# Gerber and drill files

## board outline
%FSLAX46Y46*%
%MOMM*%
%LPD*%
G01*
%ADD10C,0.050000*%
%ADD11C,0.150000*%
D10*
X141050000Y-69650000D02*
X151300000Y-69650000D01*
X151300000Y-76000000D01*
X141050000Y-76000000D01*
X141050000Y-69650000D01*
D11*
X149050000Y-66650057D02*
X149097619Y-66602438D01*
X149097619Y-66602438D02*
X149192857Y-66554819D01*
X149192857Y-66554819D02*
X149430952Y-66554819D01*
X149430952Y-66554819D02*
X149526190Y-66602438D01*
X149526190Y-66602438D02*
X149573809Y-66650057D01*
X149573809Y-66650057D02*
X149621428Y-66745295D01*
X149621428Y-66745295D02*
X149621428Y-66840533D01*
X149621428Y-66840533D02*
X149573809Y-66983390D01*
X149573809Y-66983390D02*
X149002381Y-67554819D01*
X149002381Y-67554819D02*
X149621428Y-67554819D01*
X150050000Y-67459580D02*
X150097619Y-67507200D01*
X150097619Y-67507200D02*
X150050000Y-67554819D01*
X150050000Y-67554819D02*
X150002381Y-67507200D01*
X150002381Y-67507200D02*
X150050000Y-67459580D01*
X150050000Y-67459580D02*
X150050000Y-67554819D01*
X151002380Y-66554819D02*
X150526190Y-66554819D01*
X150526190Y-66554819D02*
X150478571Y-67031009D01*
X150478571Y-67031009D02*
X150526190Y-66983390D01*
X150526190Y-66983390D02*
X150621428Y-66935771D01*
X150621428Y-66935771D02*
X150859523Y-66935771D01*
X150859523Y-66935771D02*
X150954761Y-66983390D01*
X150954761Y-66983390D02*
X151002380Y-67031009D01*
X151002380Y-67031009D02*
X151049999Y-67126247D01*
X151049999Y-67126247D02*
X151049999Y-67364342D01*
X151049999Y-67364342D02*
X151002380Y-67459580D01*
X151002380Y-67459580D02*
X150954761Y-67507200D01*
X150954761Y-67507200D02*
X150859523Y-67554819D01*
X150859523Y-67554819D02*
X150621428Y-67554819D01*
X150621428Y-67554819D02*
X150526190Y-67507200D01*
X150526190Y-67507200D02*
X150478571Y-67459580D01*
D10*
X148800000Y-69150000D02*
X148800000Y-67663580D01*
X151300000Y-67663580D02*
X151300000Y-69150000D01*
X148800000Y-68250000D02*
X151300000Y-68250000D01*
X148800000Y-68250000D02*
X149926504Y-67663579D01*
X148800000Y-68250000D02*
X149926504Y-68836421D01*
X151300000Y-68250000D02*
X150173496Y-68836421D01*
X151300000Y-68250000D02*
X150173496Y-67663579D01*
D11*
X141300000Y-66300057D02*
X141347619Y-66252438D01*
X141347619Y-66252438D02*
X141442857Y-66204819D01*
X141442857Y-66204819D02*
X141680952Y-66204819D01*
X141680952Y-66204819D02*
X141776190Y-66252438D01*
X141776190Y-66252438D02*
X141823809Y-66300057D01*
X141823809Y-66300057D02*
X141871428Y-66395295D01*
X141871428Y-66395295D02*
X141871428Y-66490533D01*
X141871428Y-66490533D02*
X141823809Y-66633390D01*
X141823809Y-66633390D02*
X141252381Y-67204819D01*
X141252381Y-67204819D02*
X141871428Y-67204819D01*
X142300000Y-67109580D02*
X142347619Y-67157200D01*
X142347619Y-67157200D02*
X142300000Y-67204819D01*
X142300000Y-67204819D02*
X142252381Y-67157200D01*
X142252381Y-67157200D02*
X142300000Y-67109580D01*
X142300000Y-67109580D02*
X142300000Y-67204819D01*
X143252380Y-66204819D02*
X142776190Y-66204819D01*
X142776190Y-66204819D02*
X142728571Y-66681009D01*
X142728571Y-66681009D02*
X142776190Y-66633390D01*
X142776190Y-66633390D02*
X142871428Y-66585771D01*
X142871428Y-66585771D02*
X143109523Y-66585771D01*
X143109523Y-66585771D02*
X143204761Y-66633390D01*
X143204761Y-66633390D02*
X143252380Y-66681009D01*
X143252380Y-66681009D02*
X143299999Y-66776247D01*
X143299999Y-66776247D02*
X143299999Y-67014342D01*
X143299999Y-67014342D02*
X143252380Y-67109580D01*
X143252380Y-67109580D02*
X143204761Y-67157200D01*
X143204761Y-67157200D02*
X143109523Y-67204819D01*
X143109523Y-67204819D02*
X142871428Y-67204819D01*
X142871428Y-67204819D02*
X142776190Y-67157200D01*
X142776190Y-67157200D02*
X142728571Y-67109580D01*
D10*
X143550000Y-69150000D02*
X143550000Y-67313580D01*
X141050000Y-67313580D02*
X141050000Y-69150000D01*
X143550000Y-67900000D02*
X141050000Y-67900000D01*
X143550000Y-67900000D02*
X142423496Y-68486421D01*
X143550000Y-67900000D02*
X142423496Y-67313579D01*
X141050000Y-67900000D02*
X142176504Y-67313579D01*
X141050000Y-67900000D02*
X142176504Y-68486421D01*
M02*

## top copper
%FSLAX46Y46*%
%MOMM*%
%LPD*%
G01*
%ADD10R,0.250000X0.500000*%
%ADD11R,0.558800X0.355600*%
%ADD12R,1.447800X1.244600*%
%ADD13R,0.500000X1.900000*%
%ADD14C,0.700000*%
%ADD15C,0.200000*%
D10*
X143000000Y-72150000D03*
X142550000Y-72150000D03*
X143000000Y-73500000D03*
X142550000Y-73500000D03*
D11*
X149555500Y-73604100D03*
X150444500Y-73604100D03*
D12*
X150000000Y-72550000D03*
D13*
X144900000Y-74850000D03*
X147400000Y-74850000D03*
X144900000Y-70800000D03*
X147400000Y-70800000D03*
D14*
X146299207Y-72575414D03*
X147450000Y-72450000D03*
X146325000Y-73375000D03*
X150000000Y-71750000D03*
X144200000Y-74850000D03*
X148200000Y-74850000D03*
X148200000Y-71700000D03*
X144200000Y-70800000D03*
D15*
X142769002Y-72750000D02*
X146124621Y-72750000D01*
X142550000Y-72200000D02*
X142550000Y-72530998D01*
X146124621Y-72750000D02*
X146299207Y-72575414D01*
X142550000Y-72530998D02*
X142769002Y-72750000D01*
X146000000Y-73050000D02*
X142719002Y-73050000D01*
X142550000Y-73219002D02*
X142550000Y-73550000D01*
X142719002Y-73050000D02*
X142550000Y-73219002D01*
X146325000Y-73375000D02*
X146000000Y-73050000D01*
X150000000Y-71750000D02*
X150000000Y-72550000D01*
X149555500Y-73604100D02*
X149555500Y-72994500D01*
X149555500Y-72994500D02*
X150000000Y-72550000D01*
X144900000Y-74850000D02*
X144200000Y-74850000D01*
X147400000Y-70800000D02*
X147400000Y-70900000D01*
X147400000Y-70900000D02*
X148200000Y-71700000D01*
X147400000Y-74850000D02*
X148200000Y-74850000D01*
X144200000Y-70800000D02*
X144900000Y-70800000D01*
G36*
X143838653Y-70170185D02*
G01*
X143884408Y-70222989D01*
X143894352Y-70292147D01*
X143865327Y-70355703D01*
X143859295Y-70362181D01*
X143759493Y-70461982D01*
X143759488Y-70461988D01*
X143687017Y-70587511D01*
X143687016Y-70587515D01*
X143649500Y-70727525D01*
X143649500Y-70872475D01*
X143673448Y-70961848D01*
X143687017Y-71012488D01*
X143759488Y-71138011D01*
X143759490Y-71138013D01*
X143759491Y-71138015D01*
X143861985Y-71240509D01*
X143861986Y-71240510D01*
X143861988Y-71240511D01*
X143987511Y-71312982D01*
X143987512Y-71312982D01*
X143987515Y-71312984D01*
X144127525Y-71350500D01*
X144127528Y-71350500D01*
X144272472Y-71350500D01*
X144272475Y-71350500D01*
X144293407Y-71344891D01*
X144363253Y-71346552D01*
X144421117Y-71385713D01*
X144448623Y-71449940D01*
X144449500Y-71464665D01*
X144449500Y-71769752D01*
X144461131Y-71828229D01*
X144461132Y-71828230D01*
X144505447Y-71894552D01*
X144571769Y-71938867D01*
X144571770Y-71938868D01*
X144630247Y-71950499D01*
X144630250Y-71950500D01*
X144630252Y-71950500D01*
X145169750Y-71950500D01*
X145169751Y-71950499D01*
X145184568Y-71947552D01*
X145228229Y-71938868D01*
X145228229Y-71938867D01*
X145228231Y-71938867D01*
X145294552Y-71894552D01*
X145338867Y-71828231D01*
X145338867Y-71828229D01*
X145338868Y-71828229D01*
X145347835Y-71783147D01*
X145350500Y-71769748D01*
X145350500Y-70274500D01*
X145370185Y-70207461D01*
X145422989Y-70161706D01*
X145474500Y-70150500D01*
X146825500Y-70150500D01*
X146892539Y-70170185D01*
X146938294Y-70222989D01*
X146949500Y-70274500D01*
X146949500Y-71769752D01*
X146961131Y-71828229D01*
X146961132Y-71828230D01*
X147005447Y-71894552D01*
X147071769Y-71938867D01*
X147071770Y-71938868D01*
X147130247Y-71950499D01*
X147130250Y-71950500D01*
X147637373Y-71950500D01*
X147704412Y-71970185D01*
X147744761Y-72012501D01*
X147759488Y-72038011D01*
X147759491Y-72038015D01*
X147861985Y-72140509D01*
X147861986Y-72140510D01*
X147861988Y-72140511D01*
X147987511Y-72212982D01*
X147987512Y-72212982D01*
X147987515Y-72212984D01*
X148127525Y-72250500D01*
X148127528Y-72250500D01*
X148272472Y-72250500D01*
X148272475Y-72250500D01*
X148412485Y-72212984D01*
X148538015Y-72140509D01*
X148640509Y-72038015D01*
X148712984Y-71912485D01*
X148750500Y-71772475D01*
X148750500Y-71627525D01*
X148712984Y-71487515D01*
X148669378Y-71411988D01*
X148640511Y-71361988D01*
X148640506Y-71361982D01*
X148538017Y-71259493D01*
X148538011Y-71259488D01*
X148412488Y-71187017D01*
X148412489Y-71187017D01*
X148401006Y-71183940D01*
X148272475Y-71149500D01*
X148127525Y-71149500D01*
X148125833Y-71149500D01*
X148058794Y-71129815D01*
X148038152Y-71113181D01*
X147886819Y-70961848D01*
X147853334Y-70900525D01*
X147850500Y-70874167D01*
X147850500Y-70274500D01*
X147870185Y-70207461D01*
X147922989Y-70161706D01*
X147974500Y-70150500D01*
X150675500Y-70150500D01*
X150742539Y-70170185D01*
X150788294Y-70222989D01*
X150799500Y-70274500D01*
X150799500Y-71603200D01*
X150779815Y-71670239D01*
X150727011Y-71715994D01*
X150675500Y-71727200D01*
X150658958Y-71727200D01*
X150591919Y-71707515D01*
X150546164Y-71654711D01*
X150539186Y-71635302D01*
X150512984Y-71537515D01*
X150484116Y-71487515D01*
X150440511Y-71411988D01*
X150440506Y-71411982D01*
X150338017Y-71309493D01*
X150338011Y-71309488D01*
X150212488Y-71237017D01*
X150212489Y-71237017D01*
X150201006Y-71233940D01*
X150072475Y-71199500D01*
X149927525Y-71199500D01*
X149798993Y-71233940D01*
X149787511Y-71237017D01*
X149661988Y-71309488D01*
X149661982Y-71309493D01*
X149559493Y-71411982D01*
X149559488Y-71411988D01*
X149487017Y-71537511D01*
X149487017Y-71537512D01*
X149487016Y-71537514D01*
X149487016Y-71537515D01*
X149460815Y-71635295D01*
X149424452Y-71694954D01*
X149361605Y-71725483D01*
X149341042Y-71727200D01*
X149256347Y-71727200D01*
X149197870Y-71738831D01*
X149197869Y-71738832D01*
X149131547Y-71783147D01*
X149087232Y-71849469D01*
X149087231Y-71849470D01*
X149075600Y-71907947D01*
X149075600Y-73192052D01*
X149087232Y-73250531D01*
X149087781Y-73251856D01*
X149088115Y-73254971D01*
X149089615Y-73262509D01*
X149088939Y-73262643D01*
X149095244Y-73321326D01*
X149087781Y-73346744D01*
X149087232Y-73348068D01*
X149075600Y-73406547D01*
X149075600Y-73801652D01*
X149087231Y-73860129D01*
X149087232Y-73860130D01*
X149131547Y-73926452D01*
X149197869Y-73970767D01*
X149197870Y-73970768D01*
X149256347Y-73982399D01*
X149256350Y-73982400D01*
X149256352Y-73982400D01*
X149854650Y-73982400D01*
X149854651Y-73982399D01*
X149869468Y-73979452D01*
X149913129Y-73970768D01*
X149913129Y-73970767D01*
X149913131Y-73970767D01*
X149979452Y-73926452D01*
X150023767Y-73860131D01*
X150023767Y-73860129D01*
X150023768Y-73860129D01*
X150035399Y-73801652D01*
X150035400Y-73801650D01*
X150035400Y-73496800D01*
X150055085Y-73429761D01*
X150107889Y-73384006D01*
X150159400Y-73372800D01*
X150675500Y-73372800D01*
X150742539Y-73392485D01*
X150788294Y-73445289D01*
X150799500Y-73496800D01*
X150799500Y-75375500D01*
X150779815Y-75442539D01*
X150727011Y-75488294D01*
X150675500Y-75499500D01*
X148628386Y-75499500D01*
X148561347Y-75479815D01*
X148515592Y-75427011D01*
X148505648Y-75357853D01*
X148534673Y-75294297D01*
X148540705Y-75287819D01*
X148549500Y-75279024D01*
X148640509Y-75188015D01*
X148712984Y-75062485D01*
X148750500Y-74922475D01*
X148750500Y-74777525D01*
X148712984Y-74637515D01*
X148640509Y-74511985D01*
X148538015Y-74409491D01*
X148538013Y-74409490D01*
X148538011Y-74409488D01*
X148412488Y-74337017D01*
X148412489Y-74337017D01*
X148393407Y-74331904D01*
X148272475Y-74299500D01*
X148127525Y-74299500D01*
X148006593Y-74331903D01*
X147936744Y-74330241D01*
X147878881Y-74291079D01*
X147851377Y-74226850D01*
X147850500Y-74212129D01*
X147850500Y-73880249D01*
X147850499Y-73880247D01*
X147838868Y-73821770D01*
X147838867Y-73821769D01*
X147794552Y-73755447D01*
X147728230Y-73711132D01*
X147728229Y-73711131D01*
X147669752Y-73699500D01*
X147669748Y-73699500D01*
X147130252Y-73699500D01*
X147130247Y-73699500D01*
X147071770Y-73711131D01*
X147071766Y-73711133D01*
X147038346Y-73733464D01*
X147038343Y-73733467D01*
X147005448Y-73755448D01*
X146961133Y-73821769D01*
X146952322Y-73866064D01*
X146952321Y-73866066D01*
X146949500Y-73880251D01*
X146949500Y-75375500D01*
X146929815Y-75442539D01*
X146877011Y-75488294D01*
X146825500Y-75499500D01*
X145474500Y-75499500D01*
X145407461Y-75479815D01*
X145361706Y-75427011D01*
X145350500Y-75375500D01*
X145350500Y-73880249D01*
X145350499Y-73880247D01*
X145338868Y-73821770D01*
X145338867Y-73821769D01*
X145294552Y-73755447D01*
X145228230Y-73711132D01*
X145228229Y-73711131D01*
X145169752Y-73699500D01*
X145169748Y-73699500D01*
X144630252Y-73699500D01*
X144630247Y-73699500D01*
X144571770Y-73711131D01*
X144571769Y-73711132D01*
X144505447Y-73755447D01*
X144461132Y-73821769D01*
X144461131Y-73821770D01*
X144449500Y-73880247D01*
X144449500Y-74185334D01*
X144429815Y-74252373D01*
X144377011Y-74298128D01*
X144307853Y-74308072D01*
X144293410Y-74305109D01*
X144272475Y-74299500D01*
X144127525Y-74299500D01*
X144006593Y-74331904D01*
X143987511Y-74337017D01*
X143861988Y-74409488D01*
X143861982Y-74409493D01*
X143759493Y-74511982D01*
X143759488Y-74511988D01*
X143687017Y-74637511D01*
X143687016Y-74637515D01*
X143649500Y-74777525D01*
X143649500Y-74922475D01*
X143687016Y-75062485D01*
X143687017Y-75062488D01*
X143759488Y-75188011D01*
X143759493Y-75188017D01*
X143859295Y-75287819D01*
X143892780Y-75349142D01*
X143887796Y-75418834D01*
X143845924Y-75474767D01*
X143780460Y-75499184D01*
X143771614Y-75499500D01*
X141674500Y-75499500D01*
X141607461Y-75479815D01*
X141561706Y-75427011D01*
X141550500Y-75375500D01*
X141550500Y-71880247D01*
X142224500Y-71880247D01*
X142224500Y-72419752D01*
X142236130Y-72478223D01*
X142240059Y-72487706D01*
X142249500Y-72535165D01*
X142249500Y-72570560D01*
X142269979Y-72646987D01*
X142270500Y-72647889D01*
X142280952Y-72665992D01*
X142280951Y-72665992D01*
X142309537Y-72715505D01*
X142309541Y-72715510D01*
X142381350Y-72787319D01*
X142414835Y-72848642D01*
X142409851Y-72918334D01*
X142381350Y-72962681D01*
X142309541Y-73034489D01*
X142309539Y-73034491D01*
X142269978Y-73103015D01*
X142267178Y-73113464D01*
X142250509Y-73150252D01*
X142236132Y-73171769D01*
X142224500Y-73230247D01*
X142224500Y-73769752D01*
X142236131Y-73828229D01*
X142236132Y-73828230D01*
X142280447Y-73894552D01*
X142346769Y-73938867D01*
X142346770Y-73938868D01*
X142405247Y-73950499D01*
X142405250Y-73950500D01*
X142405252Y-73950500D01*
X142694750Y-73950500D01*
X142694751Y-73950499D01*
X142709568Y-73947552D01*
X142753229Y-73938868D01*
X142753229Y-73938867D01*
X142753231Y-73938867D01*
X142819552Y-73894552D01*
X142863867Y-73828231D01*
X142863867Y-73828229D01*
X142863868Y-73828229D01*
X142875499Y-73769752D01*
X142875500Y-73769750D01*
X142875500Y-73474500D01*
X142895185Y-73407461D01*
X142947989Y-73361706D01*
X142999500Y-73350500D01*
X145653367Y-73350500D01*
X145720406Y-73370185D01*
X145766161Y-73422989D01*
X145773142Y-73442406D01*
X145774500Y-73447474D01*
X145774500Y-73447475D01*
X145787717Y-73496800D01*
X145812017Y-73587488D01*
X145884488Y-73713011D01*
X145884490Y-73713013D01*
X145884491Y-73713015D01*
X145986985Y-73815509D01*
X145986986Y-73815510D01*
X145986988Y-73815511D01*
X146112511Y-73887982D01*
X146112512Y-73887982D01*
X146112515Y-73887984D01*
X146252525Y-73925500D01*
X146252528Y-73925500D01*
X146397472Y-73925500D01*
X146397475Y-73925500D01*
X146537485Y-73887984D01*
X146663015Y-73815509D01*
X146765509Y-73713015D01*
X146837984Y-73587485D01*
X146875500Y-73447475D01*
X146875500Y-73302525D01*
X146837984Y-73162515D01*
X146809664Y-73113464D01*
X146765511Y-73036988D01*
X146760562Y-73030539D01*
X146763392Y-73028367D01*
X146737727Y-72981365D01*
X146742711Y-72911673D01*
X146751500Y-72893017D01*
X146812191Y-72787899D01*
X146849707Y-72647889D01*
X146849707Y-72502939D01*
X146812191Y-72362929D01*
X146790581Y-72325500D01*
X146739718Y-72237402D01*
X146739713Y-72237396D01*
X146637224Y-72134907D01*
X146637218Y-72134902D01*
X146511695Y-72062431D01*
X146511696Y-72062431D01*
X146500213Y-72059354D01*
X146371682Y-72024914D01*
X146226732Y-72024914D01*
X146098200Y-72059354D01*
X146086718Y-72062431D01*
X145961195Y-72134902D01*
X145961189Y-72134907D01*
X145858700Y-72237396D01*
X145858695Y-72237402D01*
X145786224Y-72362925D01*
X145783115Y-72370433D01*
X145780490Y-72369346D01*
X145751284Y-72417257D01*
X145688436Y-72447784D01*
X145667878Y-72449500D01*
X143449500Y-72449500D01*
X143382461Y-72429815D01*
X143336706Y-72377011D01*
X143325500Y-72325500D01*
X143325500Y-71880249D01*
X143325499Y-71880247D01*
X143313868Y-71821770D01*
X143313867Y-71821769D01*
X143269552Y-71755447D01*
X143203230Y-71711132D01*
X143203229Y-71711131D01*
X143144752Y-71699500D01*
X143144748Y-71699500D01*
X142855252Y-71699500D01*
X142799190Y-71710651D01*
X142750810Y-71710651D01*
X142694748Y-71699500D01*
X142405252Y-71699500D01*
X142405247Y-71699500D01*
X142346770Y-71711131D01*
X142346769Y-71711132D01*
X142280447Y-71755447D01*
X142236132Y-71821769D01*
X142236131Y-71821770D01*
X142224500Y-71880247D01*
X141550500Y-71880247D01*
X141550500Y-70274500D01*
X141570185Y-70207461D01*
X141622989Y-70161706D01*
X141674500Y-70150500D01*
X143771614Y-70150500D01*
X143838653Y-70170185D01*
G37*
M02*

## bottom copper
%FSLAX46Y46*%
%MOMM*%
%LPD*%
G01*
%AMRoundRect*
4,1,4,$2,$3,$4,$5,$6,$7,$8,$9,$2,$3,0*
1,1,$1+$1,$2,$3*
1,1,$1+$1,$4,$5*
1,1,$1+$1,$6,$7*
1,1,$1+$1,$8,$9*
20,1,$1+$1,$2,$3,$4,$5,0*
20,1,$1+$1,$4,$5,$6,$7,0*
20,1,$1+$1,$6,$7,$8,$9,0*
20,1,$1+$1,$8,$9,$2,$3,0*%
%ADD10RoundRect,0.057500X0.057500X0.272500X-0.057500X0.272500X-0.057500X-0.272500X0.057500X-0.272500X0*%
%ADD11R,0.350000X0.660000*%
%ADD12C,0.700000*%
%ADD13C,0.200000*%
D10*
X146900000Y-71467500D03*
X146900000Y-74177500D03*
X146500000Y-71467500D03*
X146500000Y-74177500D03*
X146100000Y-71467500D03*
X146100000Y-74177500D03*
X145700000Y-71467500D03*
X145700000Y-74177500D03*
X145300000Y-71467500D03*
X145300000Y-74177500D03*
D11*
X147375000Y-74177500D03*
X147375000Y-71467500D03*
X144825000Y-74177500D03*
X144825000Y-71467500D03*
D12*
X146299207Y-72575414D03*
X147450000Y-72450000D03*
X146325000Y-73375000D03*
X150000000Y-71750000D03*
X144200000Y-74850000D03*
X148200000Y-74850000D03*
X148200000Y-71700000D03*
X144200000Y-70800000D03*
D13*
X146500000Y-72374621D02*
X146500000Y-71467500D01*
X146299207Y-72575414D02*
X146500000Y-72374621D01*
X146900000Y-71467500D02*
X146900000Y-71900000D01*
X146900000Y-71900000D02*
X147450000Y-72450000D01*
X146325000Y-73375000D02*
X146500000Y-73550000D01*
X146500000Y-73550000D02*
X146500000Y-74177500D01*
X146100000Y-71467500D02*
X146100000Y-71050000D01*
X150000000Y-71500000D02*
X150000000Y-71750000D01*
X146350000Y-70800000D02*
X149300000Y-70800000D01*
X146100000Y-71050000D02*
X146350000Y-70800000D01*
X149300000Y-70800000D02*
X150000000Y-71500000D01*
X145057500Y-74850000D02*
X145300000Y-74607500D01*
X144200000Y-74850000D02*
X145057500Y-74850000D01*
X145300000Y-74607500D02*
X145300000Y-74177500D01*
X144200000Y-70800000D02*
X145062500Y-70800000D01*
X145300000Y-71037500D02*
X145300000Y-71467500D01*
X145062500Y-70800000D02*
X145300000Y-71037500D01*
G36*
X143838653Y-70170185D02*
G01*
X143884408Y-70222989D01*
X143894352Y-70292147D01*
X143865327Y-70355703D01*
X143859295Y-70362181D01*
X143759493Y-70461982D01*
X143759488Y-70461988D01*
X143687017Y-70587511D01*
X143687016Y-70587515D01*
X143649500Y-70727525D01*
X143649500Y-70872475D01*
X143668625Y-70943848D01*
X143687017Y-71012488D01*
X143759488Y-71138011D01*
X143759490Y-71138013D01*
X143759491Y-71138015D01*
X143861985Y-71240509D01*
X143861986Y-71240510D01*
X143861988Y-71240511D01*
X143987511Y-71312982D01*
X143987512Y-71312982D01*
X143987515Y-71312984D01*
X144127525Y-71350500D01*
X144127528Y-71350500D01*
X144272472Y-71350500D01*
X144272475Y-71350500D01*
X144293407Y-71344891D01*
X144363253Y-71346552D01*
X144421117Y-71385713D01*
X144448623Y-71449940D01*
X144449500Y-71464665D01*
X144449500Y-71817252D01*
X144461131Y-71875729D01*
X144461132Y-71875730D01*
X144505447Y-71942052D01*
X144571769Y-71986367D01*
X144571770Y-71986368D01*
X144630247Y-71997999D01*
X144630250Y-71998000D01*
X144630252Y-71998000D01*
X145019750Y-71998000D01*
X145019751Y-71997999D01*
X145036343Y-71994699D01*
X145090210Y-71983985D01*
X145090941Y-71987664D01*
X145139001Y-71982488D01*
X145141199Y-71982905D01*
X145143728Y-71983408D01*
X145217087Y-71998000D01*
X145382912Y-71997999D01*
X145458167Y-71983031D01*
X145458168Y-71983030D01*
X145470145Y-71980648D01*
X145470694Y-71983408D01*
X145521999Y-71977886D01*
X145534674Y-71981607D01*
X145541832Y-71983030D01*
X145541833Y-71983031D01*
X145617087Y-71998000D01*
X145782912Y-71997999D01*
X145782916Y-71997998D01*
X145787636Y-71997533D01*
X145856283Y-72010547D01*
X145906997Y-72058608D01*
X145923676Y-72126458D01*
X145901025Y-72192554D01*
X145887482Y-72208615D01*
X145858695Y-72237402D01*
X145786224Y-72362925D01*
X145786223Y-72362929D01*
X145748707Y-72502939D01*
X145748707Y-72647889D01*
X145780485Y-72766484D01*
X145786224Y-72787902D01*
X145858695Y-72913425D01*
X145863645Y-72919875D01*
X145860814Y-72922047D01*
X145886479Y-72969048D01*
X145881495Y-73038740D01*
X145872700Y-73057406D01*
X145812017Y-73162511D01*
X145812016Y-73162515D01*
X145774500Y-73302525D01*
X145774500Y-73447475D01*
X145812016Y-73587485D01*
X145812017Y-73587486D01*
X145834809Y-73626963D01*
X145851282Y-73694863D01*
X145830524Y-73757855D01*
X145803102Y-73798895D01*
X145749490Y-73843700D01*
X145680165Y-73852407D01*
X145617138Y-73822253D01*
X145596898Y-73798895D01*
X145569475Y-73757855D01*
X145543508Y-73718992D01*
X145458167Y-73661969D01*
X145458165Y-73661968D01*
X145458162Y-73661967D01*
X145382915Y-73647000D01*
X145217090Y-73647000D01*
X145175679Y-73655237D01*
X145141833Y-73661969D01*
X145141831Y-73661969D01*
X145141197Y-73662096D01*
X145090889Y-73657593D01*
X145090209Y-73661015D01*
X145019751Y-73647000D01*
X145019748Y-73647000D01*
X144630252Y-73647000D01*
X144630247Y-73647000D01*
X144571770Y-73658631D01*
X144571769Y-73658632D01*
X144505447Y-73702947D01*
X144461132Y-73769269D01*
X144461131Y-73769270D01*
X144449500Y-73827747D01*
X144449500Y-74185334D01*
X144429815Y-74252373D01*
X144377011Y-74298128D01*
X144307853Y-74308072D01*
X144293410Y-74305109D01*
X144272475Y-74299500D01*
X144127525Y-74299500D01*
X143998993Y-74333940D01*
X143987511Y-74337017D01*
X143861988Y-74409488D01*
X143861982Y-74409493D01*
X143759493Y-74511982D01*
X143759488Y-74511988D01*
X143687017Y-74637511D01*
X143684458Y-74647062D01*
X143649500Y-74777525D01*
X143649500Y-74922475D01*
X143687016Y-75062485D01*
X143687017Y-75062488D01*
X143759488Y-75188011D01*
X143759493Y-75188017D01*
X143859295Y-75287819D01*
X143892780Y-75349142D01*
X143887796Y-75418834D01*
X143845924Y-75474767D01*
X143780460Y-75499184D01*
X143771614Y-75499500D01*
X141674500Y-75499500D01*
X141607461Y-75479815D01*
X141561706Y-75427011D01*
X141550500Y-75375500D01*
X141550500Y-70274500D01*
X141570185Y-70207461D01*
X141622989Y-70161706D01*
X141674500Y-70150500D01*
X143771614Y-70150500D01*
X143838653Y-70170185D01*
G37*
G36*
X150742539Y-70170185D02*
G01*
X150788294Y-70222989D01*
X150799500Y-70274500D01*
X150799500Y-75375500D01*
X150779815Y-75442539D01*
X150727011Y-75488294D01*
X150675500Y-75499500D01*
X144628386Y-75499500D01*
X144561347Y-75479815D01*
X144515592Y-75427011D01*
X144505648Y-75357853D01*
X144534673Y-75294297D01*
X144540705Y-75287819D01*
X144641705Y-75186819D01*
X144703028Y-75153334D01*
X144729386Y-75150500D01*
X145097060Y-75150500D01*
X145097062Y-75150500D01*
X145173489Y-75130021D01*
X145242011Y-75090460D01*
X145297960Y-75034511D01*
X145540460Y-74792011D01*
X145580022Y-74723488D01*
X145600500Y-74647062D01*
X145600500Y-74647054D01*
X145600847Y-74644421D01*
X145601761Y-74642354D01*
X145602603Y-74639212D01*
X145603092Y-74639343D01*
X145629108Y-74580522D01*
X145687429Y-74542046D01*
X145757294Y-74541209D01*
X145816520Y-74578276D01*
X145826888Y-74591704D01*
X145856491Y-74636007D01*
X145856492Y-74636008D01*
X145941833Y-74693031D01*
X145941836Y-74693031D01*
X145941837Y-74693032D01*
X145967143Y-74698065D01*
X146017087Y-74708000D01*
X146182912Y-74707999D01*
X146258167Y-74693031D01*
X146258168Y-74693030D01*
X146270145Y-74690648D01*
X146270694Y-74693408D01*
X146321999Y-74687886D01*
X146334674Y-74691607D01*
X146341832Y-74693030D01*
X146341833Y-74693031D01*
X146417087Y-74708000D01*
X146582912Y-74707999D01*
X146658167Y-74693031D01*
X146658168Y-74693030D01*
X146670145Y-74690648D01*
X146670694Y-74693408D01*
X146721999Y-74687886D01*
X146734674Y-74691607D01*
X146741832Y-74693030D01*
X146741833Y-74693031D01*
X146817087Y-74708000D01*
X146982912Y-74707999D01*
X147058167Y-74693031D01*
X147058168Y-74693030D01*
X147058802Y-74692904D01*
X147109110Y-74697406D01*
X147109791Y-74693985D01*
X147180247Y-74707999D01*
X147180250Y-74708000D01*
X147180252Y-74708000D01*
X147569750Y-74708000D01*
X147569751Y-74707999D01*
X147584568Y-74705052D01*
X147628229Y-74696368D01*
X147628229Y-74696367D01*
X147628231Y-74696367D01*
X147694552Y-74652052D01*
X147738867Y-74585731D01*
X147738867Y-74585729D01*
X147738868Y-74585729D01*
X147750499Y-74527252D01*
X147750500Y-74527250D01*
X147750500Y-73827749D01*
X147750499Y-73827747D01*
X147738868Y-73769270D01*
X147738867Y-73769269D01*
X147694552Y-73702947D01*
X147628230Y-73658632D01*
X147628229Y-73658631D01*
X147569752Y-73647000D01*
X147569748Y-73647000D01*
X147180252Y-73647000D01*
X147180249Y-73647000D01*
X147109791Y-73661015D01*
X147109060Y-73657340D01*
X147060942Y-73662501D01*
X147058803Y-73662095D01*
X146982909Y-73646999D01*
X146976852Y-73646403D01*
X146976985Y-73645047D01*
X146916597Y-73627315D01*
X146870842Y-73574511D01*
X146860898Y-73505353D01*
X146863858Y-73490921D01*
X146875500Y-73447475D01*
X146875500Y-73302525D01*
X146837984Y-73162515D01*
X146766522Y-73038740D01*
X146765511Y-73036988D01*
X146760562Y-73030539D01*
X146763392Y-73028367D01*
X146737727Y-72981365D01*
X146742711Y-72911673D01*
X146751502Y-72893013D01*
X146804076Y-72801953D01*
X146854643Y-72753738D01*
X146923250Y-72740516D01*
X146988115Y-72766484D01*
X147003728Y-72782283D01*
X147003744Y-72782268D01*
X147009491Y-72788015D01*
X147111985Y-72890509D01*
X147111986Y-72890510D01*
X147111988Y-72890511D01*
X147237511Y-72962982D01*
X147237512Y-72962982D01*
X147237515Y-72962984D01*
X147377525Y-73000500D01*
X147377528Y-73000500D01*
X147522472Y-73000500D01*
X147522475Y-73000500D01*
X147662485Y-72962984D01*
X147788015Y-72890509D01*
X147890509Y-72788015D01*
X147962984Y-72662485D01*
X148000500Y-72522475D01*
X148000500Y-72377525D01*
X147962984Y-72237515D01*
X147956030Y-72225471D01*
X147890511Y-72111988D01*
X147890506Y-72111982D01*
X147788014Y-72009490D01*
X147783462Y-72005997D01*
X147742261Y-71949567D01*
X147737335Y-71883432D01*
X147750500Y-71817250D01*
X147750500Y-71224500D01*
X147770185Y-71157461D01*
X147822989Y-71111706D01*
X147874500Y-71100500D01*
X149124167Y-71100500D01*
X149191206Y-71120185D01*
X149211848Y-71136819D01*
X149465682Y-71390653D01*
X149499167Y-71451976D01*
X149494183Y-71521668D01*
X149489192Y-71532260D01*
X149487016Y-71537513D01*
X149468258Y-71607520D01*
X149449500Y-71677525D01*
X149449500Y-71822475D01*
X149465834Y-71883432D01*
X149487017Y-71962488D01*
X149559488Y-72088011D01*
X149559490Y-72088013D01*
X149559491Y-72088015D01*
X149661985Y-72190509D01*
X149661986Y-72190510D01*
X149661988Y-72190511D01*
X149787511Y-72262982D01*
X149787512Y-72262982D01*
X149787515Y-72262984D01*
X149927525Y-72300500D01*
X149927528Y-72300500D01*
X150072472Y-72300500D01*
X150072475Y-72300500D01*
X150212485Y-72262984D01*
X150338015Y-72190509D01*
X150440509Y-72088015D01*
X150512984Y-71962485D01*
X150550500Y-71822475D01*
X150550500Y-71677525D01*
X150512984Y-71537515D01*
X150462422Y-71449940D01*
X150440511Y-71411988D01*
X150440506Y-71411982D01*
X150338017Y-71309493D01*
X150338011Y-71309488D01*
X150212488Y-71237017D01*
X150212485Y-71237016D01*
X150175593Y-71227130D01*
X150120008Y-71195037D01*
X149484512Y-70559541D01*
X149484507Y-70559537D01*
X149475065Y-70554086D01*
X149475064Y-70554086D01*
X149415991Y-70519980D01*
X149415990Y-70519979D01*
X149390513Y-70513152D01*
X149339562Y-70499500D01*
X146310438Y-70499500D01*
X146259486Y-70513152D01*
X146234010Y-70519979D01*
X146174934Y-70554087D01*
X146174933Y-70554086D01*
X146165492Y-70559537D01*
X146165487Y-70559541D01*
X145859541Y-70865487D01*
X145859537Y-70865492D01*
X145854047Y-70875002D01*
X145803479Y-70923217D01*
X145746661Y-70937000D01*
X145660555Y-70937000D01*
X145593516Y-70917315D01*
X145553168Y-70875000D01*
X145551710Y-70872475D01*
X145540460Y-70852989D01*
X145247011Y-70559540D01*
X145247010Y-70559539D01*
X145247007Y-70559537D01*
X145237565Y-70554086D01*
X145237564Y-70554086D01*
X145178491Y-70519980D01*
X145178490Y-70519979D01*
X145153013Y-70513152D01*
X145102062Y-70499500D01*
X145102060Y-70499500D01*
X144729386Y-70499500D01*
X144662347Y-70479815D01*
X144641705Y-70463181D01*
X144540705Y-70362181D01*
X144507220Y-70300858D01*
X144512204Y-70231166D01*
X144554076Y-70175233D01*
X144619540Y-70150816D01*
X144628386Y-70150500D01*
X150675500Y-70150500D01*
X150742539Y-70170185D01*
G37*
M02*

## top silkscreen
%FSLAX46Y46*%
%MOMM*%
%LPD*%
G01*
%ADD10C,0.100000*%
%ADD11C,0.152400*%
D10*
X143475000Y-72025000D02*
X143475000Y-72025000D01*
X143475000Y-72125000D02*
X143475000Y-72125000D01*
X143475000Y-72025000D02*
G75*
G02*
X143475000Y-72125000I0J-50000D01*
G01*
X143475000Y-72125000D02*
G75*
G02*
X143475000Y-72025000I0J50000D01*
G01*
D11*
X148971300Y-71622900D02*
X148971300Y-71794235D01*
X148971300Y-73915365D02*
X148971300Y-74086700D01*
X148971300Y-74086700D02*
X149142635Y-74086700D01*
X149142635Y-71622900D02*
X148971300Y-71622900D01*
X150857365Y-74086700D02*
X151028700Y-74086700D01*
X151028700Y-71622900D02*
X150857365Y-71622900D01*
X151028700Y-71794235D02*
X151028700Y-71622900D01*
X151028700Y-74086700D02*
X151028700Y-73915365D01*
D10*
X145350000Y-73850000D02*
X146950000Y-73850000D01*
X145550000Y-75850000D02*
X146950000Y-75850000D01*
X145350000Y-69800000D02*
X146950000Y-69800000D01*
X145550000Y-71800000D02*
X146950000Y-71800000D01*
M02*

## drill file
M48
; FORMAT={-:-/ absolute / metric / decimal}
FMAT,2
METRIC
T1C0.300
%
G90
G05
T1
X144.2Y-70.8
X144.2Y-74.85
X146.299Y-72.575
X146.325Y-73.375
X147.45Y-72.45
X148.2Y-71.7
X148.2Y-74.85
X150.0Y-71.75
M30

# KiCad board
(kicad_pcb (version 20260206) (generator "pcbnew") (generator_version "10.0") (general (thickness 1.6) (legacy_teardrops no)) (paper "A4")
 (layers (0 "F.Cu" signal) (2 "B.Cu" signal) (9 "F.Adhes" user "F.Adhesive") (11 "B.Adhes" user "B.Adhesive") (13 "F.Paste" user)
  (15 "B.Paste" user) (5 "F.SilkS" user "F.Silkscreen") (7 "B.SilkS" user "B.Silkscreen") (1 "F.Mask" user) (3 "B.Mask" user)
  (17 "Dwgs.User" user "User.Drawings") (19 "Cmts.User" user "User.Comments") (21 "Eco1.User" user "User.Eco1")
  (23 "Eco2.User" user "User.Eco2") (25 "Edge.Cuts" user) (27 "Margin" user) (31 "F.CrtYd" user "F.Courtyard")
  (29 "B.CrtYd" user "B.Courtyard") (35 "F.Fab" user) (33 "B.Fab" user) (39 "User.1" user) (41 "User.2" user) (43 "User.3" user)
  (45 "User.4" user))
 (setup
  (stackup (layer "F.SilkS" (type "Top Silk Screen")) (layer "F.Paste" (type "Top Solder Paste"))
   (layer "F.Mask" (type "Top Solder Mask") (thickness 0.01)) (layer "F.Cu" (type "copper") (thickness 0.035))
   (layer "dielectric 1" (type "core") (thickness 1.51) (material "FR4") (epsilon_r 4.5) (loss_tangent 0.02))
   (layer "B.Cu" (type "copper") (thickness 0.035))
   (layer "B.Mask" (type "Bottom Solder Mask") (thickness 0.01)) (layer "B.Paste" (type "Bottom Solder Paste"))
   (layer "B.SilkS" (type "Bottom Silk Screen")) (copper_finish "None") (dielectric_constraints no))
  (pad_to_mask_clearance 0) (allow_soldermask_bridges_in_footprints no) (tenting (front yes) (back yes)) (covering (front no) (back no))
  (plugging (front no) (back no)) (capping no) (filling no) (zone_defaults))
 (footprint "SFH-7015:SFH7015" (layer "F.Cu") (at 142.775 72.825 90)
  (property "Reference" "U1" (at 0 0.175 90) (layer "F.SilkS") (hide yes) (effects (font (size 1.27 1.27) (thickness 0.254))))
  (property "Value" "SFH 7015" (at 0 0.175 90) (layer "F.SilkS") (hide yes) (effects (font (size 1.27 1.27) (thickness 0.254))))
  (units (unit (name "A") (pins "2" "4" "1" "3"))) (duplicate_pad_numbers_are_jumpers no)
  (fp_line (start 0.8 0.7) (end 0.8 0.7) (stroke (width 0.1) (type solid)) (layer "F.SilkS"))
  (fp_line (start 0.7 0.7) (end 0.7 0.7) (stroke (width 0.1) (type solid)) (layer "F.SilkS"))
  (fp_arc (start 0.8 0.7) (mid 0.75 0.75) (end 0.7 0.7) (stroke (width 0.1) (type solid)) (layer "F.SilkS"))
  (fp_arc (start 0.7 0.7) (mid 0.75 0.65) (end 0.8 0.7) (stroke (width 0.1) (type solid)) (layer "F.SilkS"))
  (pad "1" smd rect (at 0.675 0.225 180) (size 0.25 0.5) (layers "F.Cu" "F.Mask" "F.Paste") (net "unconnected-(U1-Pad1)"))
  (pad "2" smd rect (at 0.675 -0.225 180) (size 0.25 0.5) (layers "F.Cu" "F.Mask" "F.Paste") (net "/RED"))
  (pad "3" smd rect (at -0.675 0.225 180) (size 0.25 0.5) (layers "F.Cu" "F.Mask" "F.Paste") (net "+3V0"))
  (pad "4" smd rect (at -0.675 -0.225 180) (size 0.25 0.5) (layers "F.Cu" "F.Mask" "F.Paste") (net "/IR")))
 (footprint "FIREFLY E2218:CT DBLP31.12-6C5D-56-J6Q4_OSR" (layer "F.Cu") (at 150 72.8548 90)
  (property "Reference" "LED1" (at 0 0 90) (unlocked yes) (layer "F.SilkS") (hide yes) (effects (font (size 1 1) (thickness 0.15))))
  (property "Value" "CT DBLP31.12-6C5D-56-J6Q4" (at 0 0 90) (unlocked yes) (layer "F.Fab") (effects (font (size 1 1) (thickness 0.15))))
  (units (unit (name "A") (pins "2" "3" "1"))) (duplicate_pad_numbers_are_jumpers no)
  (fp_line (start 1.2319 -1.0287) (end 1.060565 -1.0287) (stroke (width 0.1524) (type solid)) (layer "F.SilkS"))
  (fp_line (start -1.060565 -1.0287) (end -1.2319 -1.0287) (stroke (width 0.1524) (type solid)) (layer "F.SilkS"))
  (fp_line (start -1.2319 -1.0287) (end -1.2319 -0.857365) (stroke (width 0.1524) (type solid)) (layer "F.SilkS"))
  (fp_line (start 1.2319 -0.857365) (end 1.2319 -1.0287) (stroke (width 0.1524) (type solid)) (layer "F.SilkS"))
  (fp_line (start -1.2319 0.857365) (end -1.2319 1.0287) (stroke (width 0.1524) (type solid)) (layer "F.SilkS"))
  (fp_line (start 1.2319 1.0287) (end 1.2319 0.857365) (stroke (width 0.1524) (type solid)) (layer "F.SilkS"))
  (fp_line (start 1.060565 1.0287) (end 1.2319 1.0287) (stroke (width 0.1524) (type solid)) (layer "F.SilkS"))
  (fp_line (start -1.2319 1.0287) (end -1.060565 1.0287) (stroke (width 0.1524) (type solid)) (layer "F.SilkS"))
  (pad "1" smd rect (at -0.7493 -0.4445 90) (size 0.3556 0.5588) (layers "F.Cu" "F.Mask" "F.Paste") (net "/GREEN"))
  (pad "2" smd rect (at -0.7493 0.4445 90) (size 0.3556 0.5588) (layers "F.Cu" "F.Mask" "F.Paste") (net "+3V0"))
  (pad "3" smd rect (at 0.3048 0 90) (size 1.2446 1.4478) (layers "F.Cu" "F.Mask" "F.Paste") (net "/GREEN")))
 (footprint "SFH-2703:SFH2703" (layer "F.Cu") (at 146.15 74.85)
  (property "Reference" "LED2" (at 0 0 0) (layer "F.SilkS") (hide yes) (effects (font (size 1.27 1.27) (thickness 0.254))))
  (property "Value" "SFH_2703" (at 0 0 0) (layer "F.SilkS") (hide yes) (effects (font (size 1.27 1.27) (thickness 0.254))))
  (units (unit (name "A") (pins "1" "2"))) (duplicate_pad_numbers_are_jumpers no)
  (fp_line (start -0.8 -1) (end 0.8 -1) (stroke (width 0.1) (type solid)) (layer "F.SilkS"))
  (fp_line (start -0.6 1) (end 0.8 1) (stroke (width 0.1) (type solid)) (layer "F.SilkS"))
  (pad "1" smd rect (at -1.25 0) (size 0.5 1.9) (layers "F.Cu" "F.Mask" "F.Paste") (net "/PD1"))
  (pad "2" smd rect (at 1.25 0) (size 0.5 1.9) (layers "F.Cu" "F.Mask" "F.Paste") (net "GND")))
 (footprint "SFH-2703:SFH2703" (layer "F.Cu") (at 146.15 70.8)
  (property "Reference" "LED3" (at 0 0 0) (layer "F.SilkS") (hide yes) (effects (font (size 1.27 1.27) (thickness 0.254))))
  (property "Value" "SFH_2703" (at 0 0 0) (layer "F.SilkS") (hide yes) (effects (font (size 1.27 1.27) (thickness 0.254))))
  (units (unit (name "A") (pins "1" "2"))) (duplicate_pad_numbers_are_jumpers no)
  (fp_line (start -0.8 -1) (end 0.8 -1) (stroke (width 0.1) (type solid)) (layer "F.SilkS"))
  (fp_line (start -0.6 1) (end 0.8 1) (stroke (width 0.1) (type solid)) (layer "F.SilkS"))
  (pad "1" smd rect (at -1.25 0) (size 0.5 1.9) (layers "F.Cu" "F.Mask" "F.Paste") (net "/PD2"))
  (pad "2" smd rect (at 1.25 0) (size 0.5 1.9) (layers "F.Cu" "F.Mask" "F.Paste") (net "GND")))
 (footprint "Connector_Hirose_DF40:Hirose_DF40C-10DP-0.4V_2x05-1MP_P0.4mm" (layer "B.Cu") (at 146.1 72.8225 180)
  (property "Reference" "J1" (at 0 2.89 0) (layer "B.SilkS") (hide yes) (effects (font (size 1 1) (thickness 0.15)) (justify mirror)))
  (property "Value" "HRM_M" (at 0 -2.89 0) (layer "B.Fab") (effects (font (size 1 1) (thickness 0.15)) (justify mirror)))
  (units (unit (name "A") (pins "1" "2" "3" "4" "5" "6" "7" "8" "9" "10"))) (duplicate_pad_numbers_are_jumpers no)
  (pad "1" smd roundrect (at -0.8 1.355 180) (size 0.23 0.66) (layers "B.Cu" "B.Mask" "B.Paste") (roundrect_rratio 0.25) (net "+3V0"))
  (pad "2" smd roundrect (at -0.8 -1.355 180) (size 0.23 0.66) (layers "B.Cu" "B.Mask" "B.Paste") (roundrect_rratio 0.25)
   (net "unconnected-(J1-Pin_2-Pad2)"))
  (pad "3" smd roundrect (at -0.4 1.355 180) (size 0.23 0.66) (layers "B.Cu" "B.Mask" "B.Paste") (roundrect_rratio 0.25) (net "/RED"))
  (pad "4" smd roundrect (at -0.4 -1.355 180) (size 0.23 0.66) (layers "B.Cu" "B.Mask" "B.Paste") (roundrect_rratio 0.25) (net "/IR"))
  (pad "5" smd roundrect (at 0 1.355 180) (size 0.23 0.66) (layers "B.Cu" "B.Mask" "B.Paste") (roundrect_rratio 0.25) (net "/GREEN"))
  (pad "6" smd roundrect (at 0 -1.355 180) (size 0.23 0.66) (layers "B.Cu" "B.Mask" "B.Paste") (roundrect_rratio 0.25)
   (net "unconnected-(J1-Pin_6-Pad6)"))
  (pad "7" smd roundrect (at 0.4 1.355 180) (size 0.23 0.66) (layers "B.Cu" "B.Mask" "B.Paste") (roundrect_rratio 0.25)
   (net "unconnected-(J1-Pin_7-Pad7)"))
  (pad "8" smd roundrect (at 0.4 -1.355 180) (size 0.23 0.66) (layers "B.Cu" "B.Mask" "B.Paste") (roundrect_rratio 0.25) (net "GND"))
  (pad "9" smd roundrect (at 0.8 1.355 180) (size 0.23 0.66) (layers "B.Cu" "B.Mask" "B.Paste") (roundrect_rratio 0.25) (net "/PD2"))
  (pad "10" smd roundrect (at 0.8 -1.355 180) (size 0.23 0.66) (layers "B.Cu" "B.Mask" "B.Paste") (roundrect_rratio 0.25) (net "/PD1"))
  (pad "MP" smd rect (at -1.275 -1.355 180) (size 0.35 0.66) (layers "B.Cu" "B.Mask" "B.Paste"))
  (pad "MP" smd rect (at -1.275 1.355 180) (size 0.35 0.66) (layers "B.Cu" "B.Mask" "B.Paste"))
  (pad "MP" smd rect (at 1.275 -1.355 180) (size 0.35 0.66) (layers "B.Cu" "B.Mask" "B.Paste"))
  (pad "MP" smd rect (at 1.275 1.355 180) (size 0.35 0.66) (layers "B.Cu" "B.Mask" "B.Paste")))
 (gr_rect (start 141.05 69.65) (end 151.3 76) (stroke (width 0.05) (type default)) (fill no) (layer "Edge.Cuts"))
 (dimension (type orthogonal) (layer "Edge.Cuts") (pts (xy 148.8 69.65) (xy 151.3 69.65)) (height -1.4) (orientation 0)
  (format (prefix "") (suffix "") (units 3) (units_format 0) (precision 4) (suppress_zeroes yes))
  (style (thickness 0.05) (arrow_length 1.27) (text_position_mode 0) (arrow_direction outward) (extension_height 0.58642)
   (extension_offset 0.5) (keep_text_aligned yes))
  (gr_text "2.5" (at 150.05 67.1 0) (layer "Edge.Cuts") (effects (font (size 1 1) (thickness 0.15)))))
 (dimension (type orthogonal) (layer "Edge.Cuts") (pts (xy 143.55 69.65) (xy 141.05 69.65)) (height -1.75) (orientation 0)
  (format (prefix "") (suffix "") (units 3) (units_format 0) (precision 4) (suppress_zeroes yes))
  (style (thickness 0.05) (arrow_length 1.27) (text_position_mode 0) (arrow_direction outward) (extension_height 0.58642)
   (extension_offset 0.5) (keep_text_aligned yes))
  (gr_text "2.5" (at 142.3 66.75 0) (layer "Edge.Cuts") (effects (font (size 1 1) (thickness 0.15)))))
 (segment (start 142.769002 72.75) (end 146.124621 72.75) (width 0.2) (layer "F.Cu") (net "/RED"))
 (segment (start 142.55 72.2) (end 142.55 72.530998) (width 0.2) (layer "F.Cu") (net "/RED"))
 (segment (start 146.124621 72.75) (end 146.299207 72.575414) (width 0.2) (layer "F.Cu") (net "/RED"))
 (segment (start 142.55 72.530998) (end 142.769002 72.75) (width 0.2) (layer "F.Cu") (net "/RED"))
 (via (at 146.299207 72.575414) (size 0.7) (drill 0.3) (layers "F.Cu" "B.Cu") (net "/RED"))
 (segment (start 146.5 72.374621) (end 146.5 71.4675) (width 0.2) (layer "B.Cu") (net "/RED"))
 (segment (start 146.299207 72.575414) (end 146.5 72.374621) (width 0.2) (layer "B.Cu") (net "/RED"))
 (via (at 147.45 72.45) (size 0.7) (drill 0.3) (layers "F.Cu" "B.Cu") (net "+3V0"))
 (segment (start 146.9 71.4675) (end 146.9 71.9) (width 0.2) (layer "B.Cu") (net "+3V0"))
 (segment (start 146.9 71.9) (end 147.45 72.45) (width 0.2) (layer "B.Cu") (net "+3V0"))
 (segment (start 146 73.05) (end 142.719002 73.05) (width 0.2) (layer "F.Cu") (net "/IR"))
 (segment (start 142.55 73.219002) (end 142.55 73.55) (width 0.2) (layer "F.Cu") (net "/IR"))
 (segment (start 142.719002 73.05) (end 142.55 73.219002) (width 0.2) (layer "F.Cu") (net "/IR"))
 (segment (start 146.325 73.375) (end 146 73.05) (width 0.2) (layer "F.Cu") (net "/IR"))
 (via (at 146.325 73.375) (size 0.7) (drill 0.3) (layers "F.Cu" "B.Cu") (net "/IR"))
 (segment (start 146.325 73.375) (end 146.5 73.55) (width 0.2) (layer "B.Cu") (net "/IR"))
 (segment (start 146.5 73.55) (end 146.5 74.1775) (width 0.2) (layer "B.Cu") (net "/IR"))
 (segment (start 150 71.75) (end 150 72.55) (width 0.2) (layer "F.Cu") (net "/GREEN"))
 (segment (start 149.5555 73.6041) (end 149.5555 72.9945) (width 0.2) (layer "F.Cu") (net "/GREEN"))
 (segment (start 149.5555 72.9945) (end 150 72.55) (width 0.2) (layer "F.Cu") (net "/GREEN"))
 (via (at 150 71.75) (size 0.7) (drill 0.3) (layers "F.Cu" "B.Cu") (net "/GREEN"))
 (segment (start 146.1 71.4675) (end 146.1 71.05) (width 0.2) (layer "B.Cu") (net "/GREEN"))
 (segment (start 150 71.5) (end 150 71.75) (width 0.2) (layer "B.Cu") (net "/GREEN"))
 (segment (start 146.35 70.8) (end 149.3 70.8) (width 0.2) (layer "B.Cu") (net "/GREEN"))
 (segment (start 146.1 71.05) (end 146.35 70.8) (width 0.2) (layer "B.Cu") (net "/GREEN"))
 (segment (start 149.3 70.8) (end 150 71.5) (width 0.2) (layer "B.Cu") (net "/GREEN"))
 (segment (start 144.9 74.85) (end 144.2 74.85) (width 0.2) (layer "F.Cu") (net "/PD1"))
 (via (at 144.2 74.85) (size 0.7) (drill 0.3) (layers "F.Cu" "B.Cu") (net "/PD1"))
 (segment (start 145.0575 74.85) (end 145.3 74.6075) (width 0.2) (layer "B.Cu") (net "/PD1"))
 (segment (start 144.2 74.85) (end 145.0575 74.85) (width 0.2) (layer "B.Cu") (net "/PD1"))
 (segment (start 145.3 74.6075) (end 145.3 74.1775) (width 0.2) (layer "B.Cu") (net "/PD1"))
 (segment (start 147.4 70.8) (end 147.4 70.9) (width 0.2) (layer "F.Cu") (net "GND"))
 (segment (start 147.4 70.9) (end 148.2 71.7) (width 0.2) (layer "F.Cu") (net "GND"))
 (segment (start 147.4 74.85) (end 148.2 74.85) (width 0.2) (layer "F.Cu") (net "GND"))
 (via (at 148.2 74.85) (size 0.7) (drill 0.3) (layers "F.Cu" "B.Cu") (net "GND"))
 (via (at 148.2 71.7) (size 0.7) (drill 0.3) (layers "F.Cu" "B.Cu") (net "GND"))
 (segment (start 144.2 70.8) (end 144.9 70.8) (width 0.2) (layer "F.Cu") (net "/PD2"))
 (via (at 144.2 70.8) (size 0.7) (drill 0.3) (layers "F.Cu" "B.Cu") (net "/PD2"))
 (segment (start 144.2 70.8) (end 145.0625 70.8) (width 0.2) (layer "B.Cu") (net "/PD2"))
 (segment (start 145.3 71.0375) (end 145.3 71.4675) (width 0.2) (layer "B.Cu") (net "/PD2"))
 (segment (start 145.0625 70.8) (end 145.3 71.0375) (width 0.2) (layer "B.Cu") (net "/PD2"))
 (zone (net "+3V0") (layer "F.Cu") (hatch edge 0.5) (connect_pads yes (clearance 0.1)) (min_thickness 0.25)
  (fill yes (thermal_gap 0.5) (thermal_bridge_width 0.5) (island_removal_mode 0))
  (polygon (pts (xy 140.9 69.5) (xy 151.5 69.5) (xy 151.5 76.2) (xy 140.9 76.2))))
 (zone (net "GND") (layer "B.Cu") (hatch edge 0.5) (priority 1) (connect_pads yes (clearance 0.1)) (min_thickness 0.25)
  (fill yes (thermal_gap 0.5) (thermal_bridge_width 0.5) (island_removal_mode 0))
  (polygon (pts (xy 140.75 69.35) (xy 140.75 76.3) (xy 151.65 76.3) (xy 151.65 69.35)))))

